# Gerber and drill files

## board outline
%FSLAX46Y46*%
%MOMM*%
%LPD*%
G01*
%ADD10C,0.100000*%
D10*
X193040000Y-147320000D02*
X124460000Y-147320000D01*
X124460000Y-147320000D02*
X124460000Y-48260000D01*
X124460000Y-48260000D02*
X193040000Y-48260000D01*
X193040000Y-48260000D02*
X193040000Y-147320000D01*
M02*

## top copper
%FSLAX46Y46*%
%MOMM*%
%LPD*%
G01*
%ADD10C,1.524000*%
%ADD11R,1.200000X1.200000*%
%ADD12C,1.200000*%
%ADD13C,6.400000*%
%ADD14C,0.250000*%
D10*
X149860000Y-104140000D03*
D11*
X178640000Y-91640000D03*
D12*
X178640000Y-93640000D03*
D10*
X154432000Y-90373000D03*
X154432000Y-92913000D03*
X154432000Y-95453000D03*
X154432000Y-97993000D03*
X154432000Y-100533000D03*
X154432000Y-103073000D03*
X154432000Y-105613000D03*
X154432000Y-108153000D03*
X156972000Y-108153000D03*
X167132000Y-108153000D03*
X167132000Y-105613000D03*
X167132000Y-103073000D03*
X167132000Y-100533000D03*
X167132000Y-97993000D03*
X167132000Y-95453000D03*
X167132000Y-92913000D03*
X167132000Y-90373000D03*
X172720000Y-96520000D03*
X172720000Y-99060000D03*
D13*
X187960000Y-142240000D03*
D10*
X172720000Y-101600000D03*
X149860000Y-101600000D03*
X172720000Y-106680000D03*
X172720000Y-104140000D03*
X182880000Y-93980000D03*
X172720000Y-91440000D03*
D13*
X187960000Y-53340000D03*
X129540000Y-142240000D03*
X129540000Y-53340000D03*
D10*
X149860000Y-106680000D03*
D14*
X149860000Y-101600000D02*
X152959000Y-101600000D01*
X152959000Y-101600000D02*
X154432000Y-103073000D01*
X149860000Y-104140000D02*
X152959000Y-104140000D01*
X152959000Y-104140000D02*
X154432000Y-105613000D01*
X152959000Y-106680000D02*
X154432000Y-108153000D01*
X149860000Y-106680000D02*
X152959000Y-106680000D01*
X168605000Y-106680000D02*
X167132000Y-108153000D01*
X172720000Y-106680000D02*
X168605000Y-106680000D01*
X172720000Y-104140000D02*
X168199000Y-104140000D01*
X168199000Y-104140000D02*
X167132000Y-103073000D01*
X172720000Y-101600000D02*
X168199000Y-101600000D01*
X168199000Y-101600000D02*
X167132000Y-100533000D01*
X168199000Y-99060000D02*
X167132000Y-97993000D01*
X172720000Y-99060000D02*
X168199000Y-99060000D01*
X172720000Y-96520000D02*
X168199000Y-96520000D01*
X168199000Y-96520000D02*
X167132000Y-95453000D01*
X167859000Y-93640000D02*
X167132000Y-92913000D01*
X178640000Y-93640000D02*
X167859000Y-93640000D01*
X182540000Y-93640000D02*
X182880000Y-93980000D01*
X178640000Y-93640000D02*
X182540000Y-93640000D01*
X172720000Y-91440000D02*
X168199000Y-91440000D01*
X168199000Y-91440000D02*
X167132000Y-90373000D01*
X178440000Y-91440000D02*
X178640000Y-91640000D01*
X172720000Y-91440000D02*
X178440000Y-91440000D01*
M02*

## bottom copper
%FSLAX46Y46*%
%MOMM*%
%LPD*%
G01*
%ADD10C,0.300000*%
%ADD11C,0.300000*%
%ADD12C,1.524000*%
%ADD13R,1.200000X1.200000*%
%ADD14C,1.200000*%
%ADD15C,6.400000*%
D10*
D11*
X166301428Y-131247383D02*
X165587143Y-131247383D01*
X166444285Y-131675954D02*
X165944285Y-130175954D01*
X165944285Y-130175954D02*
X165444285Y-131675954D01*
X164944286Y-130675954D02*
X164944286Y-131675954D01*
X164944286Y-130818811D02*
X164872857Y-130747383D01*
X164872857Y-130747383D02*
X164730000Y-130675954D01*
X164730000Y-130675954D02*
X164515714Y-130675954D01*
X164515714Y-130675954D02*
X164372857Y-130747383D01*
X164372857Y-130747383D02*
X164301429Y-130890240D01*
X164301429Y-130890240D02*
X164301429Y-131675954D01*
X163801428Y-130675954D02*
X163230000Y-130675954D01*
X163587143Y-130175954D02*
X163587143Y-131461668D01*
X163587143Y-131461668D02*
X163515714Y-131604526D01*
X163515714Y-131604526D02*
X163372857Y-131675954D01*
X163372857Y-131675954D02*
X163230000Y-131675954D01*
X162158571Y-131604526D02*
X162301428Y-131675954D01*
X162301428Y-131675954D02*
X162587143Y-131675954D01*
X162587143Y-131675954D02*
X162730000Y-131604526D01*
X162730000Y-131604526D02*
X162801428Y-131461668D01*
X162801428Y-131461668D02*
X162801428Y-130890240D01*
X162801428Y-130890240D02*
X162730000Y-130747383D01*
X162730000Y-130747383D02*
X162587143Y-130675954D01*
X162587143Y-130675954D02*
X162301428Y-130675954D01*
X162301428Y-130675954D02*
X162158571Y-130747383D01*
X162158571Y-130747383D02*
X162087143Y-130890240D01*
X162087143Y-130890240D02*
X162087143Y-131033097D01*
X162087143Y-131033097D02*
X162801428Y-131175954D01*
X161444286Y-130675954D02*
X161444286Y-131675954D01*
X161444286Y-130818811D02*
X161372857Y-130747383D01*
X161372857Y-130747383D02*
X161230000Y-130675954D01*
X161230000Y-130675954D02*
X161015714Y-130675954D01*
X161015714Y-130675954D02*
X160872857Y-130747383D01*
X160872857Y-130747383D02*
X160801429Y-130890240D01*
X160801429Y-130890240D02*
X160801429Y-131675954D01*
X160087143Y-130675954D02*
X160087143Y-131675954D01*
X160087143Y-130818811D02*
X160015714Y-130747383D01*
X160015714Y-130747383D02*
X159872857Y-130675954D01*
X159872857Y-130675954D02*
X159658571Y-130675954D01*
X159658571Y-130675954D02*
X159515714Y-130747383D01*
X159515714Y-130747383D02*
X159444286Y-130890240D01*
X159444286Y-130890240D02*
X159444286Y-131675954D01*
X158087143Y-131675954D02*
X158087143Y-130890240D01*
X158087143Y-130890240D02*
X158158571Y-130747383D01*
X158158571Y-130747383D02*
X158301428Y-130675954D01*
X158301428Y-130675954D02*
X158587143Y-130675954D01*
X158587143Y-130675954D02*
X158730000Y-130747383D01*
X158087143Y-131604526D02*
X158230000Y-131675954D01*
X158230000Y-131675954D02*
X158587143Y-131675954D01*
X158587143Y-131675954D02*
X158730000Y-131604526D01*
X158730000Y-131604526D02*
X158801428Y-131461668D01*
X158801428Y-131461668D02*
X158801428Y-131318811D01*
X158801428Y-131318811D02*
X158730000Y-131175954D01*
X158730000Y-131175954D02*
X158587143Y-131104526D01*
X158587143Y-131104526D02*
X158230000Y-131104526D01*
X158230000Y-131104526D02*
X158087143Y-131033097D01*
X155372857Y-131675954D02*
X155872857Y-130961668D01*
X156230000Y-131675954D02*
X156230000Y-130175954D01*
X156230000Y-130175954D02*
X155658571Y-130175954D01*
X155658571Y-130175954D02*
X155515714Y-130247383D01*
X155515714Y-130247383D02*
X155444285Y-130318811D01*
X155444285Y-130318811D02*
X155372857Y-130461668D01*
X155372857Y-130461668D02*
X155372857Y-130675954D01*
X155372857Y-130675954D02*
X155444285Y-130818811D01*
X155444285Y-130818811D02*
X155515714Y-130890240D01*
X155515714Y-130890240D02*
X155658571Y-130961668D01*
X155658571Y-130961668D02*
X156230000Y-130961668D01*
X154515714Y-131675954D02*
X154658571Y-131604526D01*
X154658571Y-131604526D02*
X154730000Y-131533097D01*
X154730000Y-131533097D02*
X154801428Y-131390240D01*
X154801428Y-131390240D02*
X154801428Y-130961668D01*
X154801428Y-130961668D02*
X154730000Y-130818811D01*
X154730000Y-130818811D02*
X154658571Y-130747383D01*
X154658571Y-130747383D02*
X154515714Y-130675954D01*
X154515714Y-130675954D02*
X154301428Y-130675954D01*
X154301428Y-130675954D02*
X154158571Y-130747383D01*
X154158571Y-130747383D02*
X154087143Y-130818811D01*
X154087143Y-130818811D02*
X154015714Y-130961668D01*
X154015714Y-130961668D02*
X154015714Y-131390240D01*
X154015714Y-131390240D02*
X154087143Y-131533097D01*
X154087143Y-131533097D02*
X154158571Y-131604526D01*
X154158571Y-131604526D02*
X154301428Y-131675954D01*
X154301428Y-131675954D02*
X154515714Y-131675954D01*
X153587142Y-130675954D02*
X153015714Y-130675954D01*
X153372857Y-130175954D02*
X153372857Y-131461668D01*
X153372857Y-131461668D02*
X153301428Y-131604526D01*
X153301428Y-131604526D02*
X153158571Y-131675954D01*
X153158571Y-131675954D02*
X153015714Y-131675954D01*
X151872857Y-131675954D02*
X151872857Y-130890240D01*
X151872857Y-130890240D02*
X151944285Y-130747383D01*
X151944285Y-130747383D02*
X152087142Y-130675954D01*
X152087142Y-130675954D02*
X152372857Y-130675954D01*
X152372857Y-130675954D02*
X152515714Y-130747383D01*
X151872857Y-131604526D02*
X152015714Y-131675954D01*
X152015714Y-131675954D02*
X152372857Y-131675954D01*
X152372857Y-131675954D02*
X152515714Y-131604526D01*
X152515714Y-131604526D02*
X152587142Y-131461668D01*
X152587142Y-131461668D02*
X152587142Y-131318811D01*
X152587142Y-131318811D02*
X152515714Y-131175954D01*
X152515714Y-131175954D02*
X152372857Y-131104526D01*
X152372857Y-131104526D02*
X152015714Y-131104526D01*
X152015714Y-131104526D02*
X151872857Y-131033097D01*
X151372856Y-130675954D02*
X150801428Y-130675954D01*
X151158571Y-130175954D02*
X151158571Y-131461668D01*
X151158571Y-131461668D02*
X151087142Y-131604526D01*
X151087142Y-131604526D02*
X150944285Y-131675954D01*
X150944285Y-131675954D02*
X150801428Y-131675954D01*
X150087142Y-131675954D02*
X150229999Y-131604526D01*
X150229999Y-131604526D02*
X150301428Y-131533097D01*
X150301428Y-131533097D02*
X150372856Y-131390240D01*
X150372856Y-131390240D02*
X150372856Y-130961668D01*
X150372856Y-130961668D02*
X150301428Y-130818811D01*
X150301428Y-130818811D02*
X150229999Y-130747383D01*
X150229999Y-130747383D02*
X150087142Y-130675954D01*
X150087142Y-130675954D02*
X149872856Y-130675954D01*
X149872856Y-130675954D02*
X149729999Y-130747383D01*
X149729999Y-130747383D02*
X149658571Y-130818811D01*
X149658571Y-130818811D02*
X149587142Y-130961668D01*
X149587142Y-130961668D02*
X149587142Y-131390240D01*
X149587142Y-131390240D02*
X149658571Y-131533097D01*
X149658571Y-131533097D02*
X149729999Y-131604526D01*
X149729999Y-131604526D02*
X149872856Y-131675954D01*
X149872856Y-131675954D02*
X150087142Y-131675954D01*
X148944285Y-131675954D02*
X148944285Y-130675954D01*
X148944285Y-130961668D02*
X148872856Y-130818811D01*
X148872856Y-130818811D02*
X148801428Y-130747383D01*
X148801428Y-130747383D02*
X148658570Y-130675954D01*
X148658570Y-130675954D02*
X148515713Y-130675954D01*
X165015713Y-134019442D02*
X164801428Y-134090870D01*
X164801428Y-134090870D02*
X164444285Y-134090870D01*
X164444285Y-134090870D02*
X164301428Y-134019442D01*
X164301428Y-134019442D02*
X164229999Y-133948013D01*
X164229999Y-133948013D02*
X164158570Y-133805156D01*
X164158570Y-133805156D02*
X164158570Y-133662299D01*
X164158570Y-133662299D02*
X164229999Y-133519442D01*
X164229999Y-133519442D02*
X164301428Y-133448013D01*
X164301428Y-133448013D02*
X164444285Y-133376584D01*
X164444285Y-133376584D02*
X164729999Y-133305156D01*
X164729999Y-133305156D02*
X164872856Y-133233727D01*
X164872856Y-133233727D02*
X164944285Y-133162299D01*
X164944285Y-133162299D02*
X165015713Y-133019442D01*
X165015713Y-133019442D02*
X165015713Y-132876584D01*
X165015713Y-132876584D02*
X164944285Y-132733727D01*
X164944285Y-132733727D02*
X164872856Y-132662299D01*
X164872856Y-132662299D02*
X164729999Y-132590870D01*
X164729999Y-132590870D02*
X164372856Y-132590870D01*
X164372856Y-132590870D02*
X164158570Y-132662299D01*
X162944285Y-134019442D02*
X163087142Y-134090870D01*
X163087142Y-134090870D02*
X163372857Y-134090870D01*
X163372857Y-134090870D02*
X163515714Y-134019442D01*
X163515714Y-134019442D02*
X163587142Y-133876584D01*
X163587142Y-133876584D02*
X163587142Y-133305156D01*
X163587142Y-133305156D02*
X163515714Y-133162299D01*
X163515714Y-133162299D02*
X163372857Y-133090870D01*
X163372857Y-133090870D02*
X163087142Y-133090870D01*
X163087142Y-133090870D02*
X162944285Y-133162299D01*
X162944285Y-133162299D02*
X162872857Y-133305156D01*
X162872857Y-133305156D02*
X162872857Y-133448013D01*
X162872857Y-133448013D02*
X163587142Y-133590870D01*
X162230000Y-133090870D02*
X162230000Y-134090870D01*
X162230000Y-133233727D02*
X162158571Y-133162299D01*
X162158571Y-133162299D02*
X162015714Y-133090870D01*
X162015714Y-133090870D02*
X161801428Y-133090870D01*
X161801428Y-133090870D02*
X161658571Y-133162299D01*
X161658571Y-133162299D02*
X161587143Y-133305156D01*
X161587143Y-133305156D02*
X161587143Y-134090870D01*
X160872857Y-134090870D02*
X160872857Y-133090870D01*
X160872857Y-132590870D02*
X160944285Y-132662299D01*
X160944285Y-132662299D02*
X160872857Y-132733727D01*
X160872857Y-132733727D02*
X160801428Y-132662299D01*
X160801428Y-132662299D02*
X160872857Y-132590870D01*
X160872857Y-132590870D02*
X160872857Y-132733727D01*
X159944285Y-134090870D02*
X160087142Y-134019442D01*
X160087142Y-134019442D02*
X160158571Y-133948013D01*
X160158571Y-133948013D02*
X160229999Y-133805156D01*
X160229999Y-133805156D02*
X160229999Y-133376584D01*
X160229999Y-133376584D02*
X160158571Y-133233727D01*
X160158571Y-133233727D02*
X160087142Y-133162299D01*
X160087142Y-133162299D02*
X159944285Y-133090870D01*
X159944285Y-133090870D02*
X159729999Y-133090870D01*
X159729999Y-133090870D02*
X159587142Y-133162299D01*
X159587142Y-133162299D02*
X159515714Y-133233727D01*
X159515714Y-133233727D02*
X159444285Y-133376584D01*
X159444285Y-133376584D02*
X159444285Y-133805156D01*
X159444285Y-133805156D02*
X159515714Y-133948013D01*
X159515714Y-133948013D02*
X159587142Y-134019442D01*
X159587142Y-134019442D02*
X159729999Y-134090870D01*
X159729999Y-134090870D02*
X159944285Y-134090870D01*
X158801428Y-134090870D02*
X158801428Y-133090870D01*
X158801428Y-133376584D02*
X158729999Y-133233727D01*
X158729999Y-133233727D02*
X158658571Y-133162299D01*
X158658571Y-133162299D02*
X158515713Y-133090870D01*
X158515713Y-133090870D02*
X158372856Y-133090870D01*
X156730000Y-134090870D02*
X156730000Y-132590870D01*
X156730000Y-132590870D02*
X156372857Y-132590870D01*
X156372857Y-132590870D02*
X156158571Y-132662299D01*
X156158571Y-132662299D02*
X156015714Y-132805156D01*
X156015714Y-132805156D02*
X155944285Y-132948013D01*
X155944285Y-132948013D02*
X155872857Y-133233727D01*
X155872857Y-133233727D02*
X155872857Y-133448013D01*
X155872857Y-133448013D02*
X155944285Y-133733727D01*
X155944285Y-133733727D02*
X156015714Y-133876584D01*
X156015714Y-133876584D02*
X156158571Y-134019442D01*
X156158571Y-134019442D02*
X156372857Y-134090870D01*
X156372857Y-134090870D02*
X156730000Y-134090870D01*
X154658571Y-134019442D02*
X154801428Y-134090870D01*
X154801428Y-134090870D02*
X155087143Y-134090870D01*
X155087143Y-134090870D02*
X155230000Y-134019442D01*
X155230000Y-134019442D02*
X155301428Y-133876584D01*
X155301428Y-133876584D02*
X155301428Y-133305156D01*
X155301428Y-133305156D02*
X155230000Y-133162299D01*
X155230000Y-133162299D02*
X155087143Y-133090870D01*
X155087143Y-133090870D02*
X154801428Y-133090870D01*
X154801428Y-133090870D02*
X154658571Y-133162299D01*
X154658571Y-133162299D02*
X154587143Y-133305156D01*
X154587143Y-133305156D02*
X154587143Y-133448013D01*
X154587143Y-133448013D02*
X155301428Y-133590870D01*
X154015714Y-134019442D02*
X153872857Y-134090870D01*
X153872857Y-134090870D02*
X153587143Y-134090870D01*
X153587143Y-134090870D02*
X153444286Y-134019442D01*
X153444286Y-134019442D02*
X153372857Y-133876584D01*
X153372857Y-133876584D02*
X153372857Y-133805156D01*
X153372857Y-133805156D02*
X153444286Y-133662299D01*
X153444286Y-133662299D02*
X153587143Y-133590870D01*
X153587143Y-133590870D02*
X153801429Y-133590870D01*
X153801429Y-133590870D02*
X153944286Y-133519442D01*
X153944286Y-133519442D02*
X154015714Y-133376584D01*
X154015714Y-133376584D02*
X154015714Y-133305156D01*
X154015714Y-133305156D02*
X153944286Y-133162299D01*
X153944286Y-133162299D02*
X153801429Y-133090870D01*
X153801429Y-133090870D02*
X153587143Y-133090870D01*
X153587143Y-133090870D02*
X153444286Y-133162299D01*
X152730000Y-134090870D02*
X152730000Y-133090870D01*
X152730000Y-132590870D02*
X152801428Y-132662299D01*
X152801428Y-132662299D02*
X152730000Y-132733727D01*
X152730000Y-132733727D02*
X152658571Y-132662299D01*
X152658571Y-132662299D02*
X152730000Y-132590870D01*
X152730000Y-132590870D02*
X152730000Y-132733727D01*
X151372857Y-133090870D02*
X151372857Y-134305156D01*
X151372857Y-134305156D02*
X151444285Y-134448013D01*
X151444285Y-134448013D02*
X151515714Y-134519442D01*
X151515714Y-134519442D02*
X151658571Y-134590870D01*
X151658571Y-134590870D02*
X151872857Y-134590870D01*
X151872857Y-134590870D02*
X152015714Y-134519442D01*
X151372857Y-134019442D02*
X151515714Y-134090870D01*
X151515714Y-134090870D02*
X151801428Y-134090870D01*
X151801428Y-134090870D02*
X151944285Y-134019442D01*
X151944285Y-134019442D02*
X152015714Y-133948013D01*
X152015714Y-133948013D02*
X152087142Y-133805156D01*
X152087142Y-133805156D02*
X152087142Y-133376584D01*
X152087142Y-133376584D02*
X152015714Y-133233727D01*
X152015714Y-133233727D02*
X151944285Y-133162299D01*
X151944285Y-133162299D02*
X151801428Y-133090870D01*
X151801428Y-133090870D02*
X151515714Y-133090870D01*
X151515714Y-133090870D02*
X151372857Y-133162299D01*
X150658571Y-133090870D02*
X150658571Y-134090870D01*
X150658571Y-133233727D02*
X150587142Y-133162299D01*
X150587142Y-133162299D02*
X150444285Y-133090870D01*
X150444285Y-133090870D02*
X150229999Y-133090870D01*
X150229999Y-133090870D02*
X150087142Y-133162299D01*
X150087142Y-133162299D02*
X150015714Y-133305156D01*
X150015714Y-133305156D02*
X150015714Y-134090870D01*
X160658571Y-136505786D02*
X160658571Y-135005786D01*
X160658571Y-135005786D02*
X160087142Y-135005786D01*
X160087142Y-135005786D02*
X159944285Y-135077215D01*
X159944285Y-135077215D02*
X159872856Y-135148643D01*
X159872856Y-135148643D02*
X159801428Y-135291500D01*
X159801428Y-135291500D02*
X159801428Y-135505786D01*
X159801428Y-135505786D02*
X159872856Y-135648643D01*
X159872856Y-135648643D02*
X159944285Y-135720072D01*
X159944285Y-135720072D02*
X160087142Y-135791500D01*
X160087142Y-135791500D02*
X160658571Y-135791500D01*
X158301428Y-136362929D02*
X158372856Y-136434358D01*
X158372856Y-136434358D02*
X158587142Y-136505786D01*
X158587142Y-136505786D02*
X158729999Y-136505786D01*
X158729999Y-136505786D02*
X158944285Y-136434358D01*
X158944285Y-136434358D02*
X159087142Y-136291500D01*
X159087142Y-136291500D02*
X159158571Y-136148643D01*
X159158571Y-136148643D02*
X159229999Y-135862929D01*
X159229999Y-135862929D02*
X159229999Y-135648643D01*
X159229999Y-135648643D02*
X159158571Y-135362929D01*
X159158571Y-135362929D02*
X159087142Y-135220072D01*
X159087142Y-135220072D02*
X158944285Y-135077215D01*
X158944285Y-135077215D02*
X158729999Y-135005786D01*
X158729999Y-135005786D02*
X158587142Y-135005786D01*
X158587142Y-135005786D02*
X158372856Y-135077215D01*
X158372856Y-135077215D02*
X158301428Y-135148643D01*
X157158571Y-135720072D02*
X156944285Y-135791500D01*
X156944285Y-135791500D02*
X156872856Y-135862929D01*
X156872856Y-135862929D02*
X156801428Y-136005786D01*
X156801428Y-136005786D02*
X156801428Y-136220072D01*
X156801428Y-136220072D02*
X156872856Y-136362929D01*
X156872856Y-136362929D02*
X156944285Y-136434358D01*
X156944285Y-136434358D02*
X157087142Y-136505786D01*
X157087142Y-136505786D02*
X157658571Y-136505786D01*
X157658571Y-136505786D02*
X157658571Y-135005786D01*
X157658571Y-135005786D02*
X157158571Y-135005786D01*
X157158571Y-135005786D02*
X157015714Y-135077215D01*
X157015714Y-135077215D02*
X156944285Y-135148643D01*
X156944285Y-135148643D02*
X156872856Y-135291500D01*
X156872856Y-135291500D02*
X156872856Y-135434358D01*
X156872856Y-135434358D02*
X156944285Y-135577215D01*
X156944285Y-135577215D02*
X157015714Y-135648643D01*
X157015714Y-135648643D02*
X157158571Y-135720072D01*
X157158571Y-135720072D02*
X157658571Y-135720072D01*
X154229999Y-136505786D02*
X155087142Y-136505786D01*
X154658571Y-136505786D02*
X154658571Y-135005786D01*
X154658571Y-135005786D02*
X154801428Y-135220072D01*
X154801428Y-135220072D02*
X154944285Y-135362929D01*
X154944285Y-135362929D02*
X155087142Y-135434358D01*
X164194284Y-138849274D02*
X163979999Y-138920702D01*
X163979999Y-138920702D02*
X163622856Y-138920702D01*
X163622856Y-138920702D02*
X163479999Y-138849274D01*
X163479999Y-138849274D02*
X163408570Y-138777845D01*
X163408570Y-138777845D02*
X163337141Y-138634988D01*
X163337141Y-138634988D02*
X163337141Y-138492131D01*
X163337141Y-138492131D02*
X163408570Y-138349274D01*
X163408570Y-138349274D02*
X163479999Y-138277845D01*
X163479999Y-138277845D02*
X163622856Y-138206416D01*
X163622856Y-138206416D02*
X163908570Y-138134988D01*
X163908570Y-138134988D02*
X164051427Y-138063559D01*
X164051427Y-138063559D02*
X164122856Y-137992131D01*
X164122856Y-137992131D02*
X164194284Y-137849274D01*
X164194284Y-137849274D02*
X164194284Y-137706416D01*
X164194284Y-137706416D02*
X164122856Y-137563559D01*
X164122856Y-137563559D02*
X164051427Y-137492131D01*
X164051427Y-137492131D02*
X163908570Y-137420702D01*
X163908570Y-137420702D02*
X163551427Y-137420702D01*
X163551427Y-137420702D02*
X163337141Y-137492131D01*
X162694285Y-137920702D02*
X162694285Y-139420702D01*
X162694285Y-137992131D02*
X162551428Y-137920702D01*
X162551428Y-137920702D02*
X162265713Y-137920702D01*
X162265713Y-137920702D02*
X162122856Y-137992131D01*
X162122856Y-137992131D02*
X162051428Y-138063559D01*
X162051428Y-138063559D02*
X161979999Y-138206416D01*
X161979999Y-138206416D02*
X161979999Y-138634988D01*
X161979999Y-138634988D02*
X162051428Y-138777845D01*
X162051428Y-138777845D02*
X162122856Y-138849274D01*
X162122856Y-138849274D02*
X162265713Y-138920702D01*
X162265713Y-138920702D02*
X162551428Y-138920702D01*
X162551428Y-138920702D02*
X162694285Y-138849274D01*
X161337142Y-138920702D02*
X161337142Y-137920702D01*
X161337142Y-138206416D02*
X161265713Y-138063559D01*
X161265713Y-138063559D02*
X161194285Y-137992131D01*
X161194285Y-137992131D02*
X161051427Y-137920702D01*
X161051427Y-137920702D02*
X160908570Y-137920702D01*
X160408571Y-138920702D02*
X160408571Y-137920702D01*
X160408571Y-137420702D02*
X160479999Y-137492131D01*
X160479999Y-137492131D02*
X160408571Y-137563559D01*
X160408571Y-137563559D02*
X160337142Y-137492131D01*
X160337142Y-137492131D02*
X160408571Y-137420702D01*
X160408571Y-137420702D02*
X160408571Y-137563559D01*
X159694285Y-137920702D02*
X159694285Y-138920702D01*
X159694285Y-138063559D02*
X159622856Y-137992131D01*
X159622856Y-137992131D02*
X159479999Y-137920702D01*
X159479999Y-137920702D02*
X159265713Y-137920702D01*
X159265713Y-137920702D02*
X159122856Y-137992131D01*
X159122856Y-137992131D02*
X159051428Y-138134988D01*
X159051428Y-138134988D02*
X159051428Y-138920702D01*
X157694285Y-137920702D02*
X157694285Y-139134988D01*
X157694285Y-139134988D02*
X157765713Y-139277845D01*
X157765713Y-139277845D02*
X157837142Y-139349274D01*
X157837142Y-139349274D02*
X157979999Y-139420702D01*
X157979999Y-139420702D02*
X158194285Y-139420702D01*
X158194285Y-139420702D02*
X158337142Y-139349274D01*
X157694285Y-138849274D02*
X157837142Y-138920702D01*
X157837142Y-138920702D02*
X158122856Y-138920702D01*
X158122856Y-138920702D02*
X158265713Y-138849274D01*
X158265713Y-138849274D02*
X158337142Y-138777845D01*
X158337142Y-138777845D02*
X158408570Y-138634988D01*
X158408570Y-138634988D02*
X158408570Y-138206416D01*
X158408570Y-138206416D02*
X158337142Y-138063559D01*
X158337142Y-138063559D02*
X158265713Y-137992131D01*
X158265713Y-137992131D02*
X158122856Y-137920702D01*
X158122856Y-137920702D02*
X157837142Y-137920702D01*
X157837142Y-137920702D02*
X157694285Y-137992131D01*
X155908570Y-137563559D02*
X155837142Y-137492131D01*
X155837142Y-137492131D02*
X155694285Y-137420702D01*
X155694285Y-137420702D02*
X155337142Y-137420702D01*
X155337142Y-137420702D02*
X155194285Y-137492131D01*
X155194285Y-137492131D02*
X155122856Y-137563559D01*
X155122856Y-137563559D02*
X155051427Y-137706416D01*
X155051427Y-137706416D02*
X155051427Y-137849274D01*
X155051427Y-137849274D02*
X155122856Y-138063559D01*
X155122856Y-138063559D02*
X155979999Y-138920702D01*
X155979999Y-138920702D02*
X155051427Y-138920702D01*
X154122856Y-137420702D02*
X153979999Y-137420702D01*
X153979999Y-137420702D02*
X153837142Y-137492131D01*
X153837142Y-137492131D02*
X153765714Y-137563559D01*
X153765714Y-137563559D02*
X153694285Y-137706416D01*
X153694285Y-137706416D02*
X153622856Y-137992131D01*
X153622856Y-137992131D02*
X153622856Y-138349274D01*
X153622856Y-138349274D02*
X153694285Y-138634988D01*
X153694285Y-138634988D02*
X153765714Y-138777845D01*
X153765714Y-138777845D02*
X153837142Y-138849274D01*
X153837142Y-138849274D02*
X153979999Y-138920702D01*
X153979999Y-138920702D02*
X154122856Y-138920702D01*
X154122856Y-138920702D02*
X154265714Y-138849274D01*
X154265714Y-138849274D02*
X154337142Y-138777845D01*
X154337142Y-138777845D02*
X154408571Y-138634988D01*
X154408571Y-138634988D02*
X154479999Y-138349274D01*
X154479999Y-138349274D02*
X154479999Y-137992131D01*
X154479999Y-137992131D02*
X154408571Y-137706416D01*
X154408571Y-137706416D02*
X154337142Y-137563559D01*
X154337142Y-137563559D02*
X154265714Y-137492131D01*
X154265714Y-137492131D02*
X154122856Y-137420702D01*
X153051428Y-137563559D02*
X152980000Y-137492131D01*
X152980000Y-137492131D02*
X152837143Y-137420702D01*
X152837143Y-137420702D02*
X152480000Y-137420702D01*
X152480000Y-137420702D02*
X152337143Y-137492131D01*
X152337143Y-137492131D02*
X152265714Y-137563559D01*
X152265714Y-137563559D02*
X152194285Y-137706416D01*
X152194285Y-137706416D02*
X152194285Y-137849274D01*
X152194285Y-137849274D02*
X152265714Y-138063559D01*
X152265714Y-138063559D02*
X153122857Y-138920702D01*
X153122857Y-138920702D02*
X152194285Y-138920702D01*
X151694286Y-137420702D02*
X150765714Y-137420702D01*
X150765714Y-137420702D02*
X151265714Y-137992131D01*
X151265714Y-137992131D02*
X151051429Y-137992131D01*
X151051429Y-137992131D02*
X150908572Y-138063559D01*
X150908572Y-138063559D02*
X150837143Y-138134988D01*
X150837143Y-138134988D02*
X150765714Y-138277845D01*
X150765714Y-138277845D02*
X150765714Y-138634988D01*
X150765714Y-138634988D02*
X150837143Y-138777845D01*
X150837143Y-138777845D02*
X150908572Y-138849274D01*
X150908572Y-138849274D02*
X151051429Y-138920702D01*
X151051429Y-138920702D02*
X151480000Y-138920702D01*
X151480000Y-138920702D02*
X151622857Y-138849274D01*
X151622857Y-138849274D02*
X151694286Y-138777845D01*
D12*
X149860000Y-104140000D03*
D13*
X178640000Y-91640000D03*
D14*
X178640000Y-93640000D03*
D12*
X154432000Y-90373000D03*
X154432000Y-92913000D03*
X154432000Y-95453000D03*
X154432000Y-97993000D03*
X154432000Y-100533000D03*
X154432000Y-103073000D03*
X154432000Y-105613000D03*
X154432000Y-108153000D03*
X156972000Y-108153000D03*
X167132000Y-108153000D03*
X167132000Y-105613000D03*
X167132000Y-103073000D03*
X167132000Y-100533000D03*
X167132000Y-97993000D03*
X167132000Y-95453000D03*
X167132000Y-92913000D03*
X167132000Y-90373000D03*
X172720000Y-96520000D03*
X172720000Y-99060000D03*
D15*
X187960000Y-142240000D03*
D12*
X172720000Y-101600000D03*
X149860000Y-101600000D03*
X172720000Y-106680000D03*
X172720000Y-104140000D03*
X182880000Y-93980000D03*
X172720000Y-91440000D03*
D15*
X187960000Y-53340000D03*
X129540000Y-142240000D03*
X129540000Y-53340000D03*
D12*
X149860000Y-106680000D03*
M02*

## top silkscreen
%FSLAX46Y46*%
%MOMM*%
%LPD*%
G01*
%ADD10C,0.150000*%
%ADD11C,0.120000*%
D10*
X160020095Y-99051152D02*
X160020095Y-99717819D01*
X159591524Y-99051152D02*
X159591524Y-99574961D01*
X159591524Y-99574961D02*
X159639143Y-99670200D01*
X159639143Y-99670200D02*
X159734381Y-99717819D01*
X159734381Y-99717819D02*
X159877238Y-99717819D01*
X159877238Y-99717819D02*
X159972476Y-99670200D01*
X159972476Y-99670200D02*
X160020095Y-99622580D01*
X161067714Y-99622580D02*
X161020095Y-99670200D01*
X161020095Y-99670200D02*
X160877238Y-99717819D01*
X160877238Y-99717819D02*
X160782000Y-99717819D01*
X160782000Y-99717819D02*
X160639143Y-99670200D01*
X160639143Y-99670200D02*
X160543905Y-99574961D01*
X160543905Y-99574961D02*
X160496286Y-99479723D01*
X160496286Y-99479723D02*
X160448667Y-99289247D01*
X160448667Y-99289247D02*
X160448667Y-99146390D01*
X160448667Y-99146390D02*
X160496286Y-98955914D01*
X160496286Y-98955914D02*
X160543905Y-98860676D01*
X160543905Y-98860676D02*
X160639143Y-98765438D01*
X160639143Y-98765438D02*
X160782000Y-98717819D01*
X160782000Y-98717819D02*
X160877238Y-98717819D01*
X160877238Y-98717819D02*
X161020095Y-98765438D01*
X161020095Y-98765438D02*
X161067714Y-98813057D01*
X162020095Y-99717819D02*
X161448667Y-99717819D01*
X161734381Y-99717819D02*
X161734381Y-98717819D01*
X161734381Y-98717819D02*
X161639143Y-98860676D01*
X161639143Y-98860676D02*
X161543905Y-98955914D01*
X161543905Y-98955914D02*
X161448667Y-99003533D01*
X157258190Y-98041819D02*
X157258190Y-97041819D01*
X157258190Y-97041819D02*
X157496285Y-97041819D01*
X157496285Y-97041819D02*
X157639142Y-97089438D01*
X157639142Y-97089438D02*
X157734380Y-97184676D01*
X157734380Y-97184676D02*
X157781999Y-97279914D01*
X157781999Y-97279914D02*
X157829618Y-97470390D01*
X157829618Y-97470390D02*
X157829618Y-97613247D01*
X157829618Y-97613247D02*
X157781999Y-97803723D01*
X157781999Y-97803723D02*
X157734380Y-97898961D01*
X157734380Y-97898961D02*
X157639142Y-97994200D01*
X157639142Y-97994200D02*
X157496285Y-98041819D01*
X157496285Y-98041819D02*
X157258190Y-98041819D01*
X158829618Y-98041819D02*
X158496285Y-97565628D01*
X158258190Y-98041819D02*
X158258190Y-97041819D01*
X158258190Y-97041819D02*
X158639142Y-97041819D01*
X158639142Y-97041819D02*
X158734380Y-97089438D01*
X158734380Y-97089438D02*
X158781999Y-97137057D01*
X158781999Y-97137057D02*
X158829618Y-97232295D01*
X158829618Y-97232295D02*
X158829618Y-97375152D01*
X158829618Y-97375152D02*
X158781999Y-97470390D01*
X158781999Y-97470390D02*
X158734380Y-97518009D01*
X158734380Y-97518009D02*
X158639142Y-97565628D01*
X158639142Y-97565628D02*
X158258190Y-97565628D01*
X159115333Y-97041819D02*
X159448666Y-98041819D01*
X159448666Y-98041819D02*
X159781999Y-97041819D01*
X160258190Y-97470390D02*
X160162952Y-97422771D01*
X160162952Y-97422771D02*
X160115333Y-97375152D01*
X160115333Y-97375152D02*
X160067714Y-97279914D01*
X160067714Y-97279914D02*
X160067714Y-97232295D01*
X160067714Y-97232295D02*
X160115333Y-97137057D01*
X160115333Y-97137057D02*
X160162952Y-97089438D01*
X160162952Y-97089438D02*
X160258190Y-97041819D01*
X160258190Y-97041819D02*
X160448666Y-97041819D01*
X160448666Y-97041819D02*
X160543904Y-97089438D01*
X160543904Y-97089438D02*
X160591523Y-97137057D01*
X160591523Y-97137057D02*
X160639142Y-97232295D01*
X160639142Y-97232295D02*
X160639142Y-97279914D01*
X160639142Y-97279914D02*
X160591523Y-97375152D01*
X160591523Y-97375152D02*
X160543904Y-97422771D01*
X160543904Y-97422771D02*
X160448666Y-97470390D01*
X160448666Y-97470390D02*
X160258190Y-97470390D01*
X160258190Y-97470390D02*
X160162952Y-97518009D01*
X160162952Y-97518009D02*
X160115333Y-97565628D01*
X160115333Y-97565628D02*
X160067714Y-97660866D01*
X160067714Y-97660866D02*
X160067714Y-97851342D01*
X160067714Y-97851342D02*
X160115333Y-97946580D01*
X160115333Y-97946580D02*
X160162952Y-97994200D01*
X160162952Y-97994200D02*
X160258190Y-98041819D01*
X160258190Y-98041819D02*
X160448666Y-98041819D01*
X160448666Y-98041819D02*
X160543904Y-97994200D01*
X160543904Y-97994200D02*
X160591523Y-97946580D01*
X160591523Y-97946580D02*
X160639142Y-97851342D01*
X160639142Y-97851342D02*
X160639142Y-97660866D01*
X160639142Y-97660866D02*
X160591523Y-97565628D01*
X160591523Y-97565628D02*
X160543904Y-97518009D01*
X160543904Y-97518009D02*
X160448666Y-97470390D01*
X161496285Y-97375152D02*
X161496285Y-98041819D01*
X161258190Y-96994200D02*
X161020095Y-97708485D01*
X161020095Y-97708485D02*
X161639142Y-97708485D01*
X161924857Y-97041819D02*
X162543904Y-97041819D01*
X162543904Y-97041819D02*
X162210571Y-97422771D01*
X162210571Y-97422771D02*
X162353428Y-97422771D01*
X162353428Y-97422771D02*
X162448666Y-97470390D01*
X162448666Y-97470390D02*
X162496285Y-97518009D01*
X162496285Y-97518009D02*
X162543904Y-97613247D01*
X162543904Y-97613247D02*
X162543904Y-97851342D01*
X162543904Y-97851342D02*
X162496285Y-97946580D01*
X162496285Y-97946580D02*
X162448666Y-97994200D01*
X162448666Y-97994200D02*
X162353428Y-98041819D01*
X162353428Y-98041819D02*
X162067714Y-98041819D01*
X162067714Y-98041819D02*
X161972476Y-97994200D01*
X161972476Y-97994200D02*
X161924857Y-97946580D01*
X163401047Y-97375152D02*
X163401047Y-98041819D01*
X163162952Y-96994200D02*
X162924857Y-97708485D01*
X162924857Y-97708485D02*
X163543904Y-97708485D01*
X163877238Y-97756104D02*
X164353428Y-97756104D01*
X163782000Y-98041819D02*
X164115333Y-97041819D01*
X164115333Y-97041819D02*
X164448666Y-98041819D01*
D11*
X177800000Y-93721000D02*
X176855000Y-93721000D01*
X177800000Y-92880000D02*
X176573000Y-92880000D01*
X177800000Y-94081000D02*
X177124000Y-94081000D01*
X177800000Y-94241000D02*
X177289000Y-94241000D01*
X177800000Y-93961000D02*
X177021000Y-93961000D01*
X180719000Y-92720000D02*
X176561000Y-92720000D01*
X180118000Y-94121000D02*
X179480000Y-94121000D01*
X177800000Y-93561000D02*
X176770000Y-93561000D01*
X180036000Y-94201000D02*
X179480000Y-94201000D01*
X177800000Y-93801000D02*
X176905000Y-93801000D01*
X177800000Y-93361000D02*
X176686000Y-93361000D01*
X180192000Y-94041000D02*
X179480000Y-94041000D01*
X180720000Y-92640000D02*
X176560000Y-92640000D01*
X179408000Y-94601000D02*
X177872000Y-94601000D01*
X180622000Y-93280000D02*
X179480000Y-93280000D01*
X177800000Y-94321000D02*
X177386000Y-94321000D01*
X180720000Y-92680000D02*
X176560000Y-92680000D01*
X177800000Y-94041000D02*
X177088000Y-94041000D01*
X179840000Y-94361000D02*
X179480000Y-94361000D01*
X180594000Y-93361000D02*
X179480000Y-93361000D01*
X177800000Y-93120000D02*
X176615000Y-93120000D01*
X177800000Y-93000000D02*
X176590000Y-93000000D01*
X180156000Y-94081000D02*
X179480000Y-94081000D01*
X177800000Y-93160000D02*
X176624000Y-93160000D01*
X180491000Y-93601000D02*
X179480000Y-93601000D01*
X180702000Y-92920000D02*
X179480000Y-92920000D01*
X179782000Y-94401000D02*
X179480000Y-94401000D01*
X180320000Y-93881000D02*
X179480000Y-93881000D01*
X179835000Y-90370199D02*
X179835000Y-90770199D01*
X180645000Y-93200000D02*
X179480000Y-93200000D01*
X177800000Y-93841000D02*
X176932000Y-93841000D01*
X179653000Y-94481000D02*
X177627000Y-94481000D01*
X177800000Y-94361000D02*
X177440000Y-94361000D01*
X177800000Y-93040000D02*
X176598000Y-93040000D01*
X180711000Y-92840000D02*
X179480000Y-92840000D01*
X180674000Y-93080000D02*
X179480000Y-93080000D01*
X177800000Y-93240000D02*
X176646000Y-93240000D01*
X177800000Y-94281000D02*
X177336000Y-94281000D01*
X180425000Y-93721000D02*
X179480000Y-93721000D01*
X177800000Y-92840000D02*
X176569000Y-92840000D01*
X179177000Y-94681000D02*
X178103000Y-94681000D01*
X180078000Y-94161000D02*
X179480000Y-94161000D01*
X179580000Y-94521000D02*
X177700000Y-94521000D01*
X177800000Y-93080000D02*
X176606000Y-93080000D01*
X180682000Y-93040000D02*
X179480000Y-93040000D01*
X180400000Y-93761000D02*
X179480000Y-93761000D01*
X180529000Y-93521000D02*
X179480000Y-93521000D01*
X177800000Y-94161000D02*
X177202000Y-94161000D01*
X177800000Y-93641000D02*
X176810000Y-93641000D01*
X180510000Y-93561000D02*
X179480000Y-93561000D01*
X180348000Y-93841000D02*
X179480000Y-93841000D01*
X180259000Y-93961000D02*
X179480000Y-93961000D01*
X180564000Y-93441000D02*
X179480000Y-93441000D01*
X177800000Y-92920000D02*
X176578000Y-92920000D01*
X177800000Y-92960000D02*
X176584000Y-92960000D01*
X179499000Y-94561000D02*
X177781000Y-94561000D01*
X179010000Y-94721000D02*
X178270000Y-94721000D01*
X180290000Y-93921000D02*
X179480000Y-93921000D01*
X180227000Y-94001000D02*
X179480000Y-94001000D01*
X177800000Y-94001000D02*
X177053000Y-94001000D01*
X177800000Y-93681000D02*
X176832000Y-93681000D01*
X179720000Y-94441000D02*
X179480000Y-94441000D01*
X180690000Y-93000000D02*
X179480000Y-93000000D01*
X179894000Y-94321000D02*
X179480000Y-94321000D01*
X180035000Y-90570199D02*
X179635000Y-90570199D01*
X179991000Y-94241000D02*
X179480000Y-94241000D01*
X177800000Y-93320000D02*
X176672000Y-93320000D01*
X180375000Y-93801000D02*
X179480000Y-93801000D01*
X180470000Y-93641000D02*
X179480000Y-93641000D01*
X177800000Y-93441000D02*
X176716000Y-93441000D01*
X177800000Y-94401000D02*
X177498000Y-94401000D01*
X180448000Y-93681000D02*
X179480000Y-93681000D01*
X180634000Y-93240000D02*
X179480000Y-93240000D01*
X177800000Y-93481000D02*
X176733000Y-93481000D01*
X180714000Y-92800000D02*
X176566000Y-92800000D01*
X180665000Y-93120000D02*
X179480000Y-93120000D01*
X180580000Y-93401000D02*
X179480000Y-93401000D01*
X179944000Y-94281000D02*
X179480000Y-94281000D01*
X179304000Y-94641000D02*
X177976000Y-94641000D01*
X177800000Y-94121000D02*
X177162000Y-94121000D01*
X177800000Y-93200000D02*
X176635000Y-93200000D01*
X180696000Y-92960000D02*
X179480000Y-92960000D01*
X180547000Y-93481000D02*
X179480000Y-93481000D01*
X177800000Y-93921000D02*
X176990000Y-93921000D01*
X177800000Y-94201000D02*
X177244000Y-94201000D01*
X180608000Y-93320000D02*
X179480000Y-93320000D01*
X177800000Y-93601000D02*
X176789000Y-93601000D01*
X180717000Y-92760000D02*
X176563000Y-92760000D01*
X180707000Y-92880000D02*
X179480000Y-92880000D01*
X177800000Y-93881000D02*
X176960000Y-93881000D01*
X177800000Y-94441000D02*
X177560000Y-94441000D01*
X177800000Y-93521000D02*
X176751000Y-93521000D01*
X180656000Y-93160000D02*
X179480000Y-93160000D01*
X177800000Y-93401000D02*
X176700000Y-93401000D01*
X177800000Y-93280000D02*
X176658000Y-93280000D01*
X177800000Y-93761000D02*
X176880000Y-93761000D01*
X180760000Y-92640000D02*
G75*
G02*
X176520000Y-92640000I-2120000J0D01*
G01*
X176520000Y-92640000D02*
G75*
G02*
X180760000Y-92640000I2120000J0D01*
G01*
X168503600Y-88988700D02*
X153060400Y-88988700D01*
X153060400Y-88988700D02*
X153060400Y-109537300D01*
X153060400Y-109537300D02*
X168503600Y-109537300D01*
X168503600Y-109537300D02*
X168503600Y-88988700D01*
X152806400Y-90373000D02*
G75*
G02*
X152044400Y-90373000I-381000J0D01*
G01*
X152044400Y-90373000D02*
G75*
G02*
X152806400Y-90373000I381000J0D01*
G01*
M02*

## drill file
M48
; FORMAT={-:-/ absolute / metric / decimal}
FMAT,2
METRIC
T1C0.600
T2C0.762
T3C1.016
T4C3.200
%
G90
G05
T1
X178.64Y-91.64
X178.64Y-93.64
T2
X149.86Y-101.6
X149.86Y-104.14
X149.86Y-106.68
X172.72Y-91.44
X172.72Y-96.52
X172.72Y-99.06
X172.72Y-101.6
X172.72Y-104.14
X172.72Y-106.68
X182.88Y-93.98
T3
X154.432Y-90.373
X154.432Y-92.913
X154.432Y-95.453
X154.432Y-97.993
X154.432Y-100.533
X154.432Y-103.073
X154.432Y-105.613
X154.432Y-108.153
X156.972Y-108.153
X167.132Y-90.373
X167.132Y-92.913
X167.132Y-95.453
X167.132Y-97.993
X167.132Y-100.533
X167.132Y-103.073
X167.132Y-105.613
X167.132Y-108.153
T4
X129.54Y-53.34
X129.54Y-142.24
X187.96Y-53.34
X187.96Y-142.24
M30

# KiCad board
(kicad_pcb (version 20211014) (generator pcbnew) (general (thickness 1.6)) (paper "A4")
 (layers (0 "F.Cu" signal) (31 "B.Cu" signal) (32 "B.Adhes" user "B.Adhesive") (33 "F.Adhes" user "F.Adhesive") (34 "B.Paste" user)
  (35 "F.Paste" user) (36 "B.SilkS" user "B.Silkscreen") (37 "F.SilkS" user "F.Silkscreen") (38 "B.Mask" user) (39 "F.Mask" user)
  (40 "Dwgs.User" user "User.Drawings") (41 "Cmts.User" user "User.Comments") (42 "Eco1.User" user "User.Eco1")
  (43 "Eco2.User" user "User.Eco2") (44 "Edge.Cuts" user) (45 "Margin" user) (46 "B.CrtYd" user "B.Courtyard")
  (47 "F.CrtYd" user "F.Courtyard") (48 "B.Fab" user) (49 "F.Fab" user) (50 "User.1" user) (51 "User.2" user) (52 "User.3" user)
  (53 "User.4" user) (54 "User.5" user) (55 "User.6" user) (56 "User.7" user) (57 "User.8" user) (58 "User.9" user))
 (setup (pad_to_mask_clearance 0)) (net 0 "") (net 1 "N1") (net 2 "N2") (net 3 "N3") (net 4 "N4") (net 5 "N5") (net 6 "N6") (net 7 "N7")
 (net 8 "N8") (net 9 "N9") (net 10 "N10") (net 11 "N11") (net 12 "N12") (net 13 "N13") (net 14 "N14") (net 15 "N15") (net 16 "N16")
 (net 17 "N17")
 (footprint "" (layer "F.Cu") (at 149.86 104.14)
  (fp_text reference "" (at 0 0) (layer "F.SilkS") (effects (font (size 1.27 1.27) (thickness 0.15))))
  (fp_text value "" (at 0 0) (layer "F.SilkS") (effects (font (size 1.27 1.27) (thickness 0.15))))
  (pad "1" thru_hole circle (at 0 0) (size 1.524 1.524) (drill 0.762) (layers *.Cu *.Mask) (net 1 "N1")))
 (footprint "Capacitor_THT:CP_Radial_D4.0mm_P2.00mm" (layer "F.Cu") (at 178.64 91.64 -90)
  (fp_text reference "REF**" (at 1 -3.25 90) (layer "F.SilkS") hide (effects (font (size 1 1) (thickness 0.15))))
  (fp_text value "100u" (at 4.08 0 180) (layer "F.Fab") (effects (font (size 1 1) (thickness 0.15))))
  (fp_line (start 2.081 0.84) (end 2.081 1.785) (layer "F.SilkS") (width 0.12))
  (fp_line (start 1.24 0.84) (end 1.24 2.067) (layer "F.SilkS") (width 0.12))
  (fp_line (start 2.441 0.84) (end 2.441 1.516) (layer "F.SilkS") (width 0.12))
  (fp_line (start 2.601 0.84) (end 2.601 1.351) (layer "F.SilkS") (width 0.12))
  (fp_line (start 2.321 0.84) (end 2.321 1.619) (layer "F.SilkS") (width 0.12))
  (fp_line (start 1.08 -2.079) (end 1.08 2.079) (layer "F.SilkS") (width 0.12))
  (fp_line (start 2.481 -1.478) (end 2.481 -0.84) (layer "F.SilkS") (width 0.12))
  (fp_line (start 1.921 0.84) (end 1.921 1.87) (layer "F.SilkS") (width 0.12))
  (fp_line (start 2.561 -1.396) (end 2.561 -0.84) (layer "F.SilkS") (width 0.12))
  (fp_line (start 2.161 0.84) (end 2.161 1.735) (layer "F.SilkS") (width 0.12))
  (fp_line (start 1.721 0.84) (end 1.721 1.954) (layer "F.SilkS") (width 0.12))
  (fp_line (start 2.401 -1.552) (end 2.401 -0.84) (layer "F.SilkS") (width 0.12))
  (fp_line (start 1 -2.08) (end 1 2.08) (layer "F.SilkS") (width 0.12))
  (fp_line (start 2.961 -0.768) (end 2.961 0.768) (layer "F.SilkS") (width 0.12))
  (fp_line (start 1.64 -1.982) (end 1.64 -0.84) (layer "F.SilkS") (width 0.12))
  (fp_line (start 2.681 0.84) (end 2.681 1.254) (layer "F.SilkS") (width 0.12))
  (fp_line (start 1.04 -2.08) (end 1.04 2.08) (layer "F.SilkS") (width 0.12))
  (fp_line (start 2.401 0.84) (end 2.401 1.552) (layer "F.SilkS") (width 0.12))
  (fp_line (start 2.721 -1.2) (end 2.721 -0.84) (layer "F.SilkS") (width 0.12))
  (fp_line (start 1.721 -1.954) (end 1.721 -0.84) (layer "F.SilkS") (width 0.12))
  (fp_line (start 1.48 0.84) (end 1.48 2.025) (layer "F.SilkS") (width 0.12))
  (fp_line (start 1.36 0.84) (end 1.36 2.05) (layer "F.SilkS") (width 0.12))
  (fp_line (start 2.441 -1.516) (end 2.441 -0.84) (layer "F.SilkS") (width 0.12))
  (fp_line (start 1.52 0.84) (end 1.52 2.016) (layer "F.SilkS") (width 0.12))
  (fp_line (start 1.961 -1.851) (end 1.961 -0.84) (layer "F.SilkS") (width 0.12))
  (fp_line (start 1.28 -2.062) (end 1.28 -0.84) (layer "F.SilkS") (width 0.12))
  (fp_line (start 2.761 -1.142) (end 2.761 -0.84) (layer "F.SilkS") (width 0.12))
  (fp_line (start 2.241 -1.68) (end 2.241 -0.84) (layer "F.SilkS") (width 0.12))
  (fp_line (start -1.269801 -1.195) (end -0.869801 -1.195) (layer "F.SilkS") (width 0.12))
  (fp_line (start 1.56 -2.005) (end 1.56 -0.84) (layer "F.SilkS") (width 0.12))
  (fp_line (start 2.201 0.84) (end 2.201 1.708) (layer "F.SilkS") (width 0.12))
  (fp_line (start 2.841 -1.013) (end 2.841 1.013) (layer "F.SilkS") (width 0.12))
  (fp_line (start 2.721 0.84) (end 2.721 1.2) (layer "F.SilkS") (width 0.12))
  (fp_line (start 1.4 0.84) (end 1.4 2.042) (layer "F.SilkS") (width 0.12))
  (fp_line (start 1.2 -2.071) (end 1.2 -0.84) (layer "F.SilkS") (width 0.12))
  (fp_line (start 1.44 -2.034) (end 1.44 -0.84) (layer "F.SilkS") (width 0.12))
  (fp_line (start 1.6 0.84) (end 1.6 1.994) (layer "F.SilkS") (width 0.12))
  (fp_line (start 2.641 0.84) (end 2.641 1.304) (layer "F.SilkS") (width 0.12))
  (fp_line (start 2.081 -1.785) (end 2.081 -0.84) (layer "F.SilkS") (width 0.12))
  (fp_line (start 1.2 0.84) (end 1.2 2.071) (layer "F.SilkS") (width 0.12))
  (fp_line (start 3.041 -0.537) (end 3.041 0.537) (layer "F.SilkS") (width 0.12))
  (fp_line (start 2.521 -1.438) (end 2.521 -0.84) (layer "F.SilkS") (width 0.12))
  (fp_line (start 2.881 -0.94) (end 2.881 0.94) (layer "F.SilkS") (width 0.12))
  (fp_line (start 1.44 0.84) (end 1.44 2.034) (layer "F.SilkS") (width 0.12))
  (fp_line (start 1.4 -2.042) (end 1.4 -0.84) (layer "F.SilkS") (width 0.12))
  (fp_line (start 2.121 -1.76) (end 2.121 -0.84) (layer "F.SilkS") (width 0.12))
  (fp_line (start 1.881 -1.889) (end 1.881 -0.84) (layer "F.SilkS") (width 0.12))
  (fp_line (start 2.521 0.84) (end 2.521 1.438) (layer "F.SilkS") (width 0.12))
  (fp_line (start 2.001 0.84) (end 2.001 1.83) (layer "F.SilkS") (width 0.12))
  (fp_line (start 1.921 -1.87) (end 1.921 -0.84) (layer "F.SilkS") (width 0.12))
  (fp_line (start 2.201 -1.708) (end 2.201 -0.84) (layer "F.SilkS") (width 0.12))
  (fp_line (start 2.321 -1.619) (end 2.321 -0.84) (layer "F.SilkS") (width 0.12))
  (fp_line (start 1.801 -1.924) (end 1.801 -0.84) (layer "F.SilkS") (width 0.12))
  (fp_line (start 1.28 0.84) (end 1.28 2.062) (layer "F.SilkS") (width 0.12))
  (fp_line (start 1.32 0.84) (end 1.32 2.056) (layer "F.SilkS") (width 0.12))
  (fp_line (start 2.921 -0.859) (end 2.921 0.859) (layer "F.SilkS") (width 0.12))
  (fp_line (start 3.081 -0.37) (end 3.081 0.37) (layer "F.SilkS") (width 0.12))
  (fp_line (start 2.281 -1.65) (end 2.281 -0.84) (layer "F.SilkS") (width 0.12))
  (fp_line (start 2.361 -1.587) (end 2.361 -0.84) (layer "F.SilkS") (width 0.12))
  (fp_line (start 2.361 0.84) (end 2.361 1.587) (layer "F.SilkS") (width 0.12))
  (fp_line (start 2.041 0.84) (end 2.041 1.808) (layer "F.SilkS") (width 0.12))
  (fp_line (start 2.801 -1.08) (end 2.801 -0.84) (layer "F.SilkS") (width 0.12))
  (fp_line (start 1.36 -2.05) (end 1.36 -0.84) (layer "F.SilkS") (width 0.12))
  (fp_line (start 2.681 -1.254) (end 2.681 -0.84) (layer "F.SilkS") (width 0.12))
  (fp_line (start -1.069801 -1.395) (end -1.069801 -0.995) (layer "F.SilkS") (width 0.12))
  (fp_line (start 2.601 -1.351) (end 2.601 -0.84) (layer "F.SilkS") (width 0.12))
  (fp_line (start 1.68 0.84) (end 1.68 1.968) (layer "F.SilkS") (width 0.12))
  (fp_line (start 2.161 -1.735) (end 2.161 -0.84) (layer "F.SilkS") (width 0.12))
  (fp_line (start 2.001 -1.83) (end 2.001 -0.84) (layer "F.SilkS") (width 0.12))
  (fp_line (start 1.801 0.84) (end 1.801 1.924) (layer "F.SilkS") (width 0.12))
  (fp_line (start 2.761 0.84) (end 2.761 1.142) (layer "F.SilkS") (width 0.12))
  (fp_line (start 2.041 -1.808) (end 2.041 -0.84) (layer "F.SilkS") (width 0.12))
  (fp_line (start 1.6 -1.994) (end 1.6 -0.84) (layer "F.SilkS") (width 0.12))
  (fp_line (start 1.841 0.84) (end 1.841 1.907) (layer "F.SilkS") (width 0.12))
  (fp_line (start 1.16 -2.074) (end 1.16 2.074) (layer "F.SilkS") (width 0.12))
  (fp_line (start 1.48 -2.025) (end 1.48 -0.84) (layer "F.SilkS") (width 0.12))
  (fp_line (start 1.761 -1.94) (end 1.761 -0.84) (layer "F.SilkS") (width 0.12))
  (fp_line (start 2.641 -1.304) (end 2.641 -0.84) (layer "F.SilkS") (width 0.12))
  (fp_line (start 3.001 -0.664) (end 3.001 0.664) (layer "F.SilkS") (width 0.12))
  (fp_line (start 2.481 0.84) (end 2.481 1.478) (layer "F.SilkS") (width 0.12))
  (fp_line (start 1.56 0.84) (end 1.56 2.005) (layer "F.SilkS") (width 0.12))
  (fp_line (start 1.32 -2.056) (end 1.32 -0.84) (layer "F.SilkS") (width 0.12))
  (fp_line (start 1.841 -1.907) (end 1.841 -0.84) (layer "F.SilkS") (width 0.12))
  (fp_line (start 2.281 0.84) (end 2.281 1.65) (layer "F.SilkS") (width 0.12))
  (fp_line (start 2.561 0.84) (end 2.561 1.396) (layer "F.SilkS") (width 0.12))
  (fp_line (start 1.68 -1.968) (end 1.68 -0.84) (layer "F.SilkS") (width 0.12))
  (fp_line (start 1.961 0.84) (end 1.961 1.851) (layer "F.SilkS") (width 0.12))
  (fp_line (start 1.12 -2.077) (end 1.12 2.077) (layer "F.SilkS") (width 0.12))
  (fp_line (start 1.24 -2.067) (end 1.24 -0.84) (layer "F.SilkS") (width 0.12))
  (fp_line (start 2.241 0.84) (end 2.241 1.68) (layer "F.SilkS") (width 0.12))
  (fp_line (start 2.801 0.84) (end 2.801 1.08) (layer "F.SilkS") (width 0.12))
  (fp_line (start 1.881 0.84) (end 1.881 1.889) (layer "F.SilkS") (width 0.12))
  (fp_line (start 1.52 -2.016) (end 1.52 -0.84) (layer "F.SilkS") (width 0.12))
  (fp_line (start 1.761 0.84) (end 1.761 1.94) (layer "F.SilkS") (width 0.12))
  (fp_line (start 1.64 0.84) (end 1.64 1.982) (layer "F.SilkS") (width 0.12))
  (fp_line (start 2.121 0.84) (end 2.121 1.76) (layer "F.SilkS") (width 0.12))
  (fp_circle (center 1 0) (end 3.12 0) (layer "F.SilkS") (width 0.12) (fill none))
  (pad "1" thru_hole rect (at 0 0 270) (size 1.2 1.2) (drill 0.6) (layers *.Cu *.Mask) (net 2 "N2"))
  (pad "2" thru_hole circle (at 2 0 270) (size 1.2 1.2) (drill 0.6) (layers *.Cu *.Mask) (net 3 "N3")))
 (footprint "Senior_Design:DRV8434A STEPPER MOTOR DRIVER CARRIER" (layer "F.Cu") (at 154.432 90.373)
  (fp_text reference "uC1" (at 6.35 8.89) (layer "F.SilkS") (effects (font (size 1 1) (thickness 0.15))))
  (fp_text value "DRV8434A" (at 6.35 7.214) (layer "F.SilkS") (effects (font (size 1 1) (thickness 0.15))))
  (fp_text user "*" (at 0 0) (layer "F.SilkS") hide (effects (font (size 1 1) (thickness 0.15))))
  (fp_line (start 14.0716 -1.3843) (end -1.3716 -1.3843) (layer "F.SilkS") (width 0.12))
  (fp_line (start -1.3716 -1.3843) (end -1.3716 19.1643) (layer "F.SilkS") (width 0.12))
  (fp_line (start -1.3716 19.1643) (end 14.0716 19.1643) (layer "F.SilkS") (width 0.12))
  (fp_line (start 14.0716 19.1643) (end 14.0716 -1.3843) (layer "F.SilkS") (width 0.12))
  (fp_circle (center -2.0066 0) (end -1.6256 0) (layer "F.SilkS") (width 0.12) (fill none))
  (pad "1" thru_hole circle (at 0 0) (size 1.524 1.524) (drill 1.016) (layers *.Cu *.Mask) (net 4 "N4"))
  (pad "2" thru_hole circle (at 0 2.54) (size 1.524 1.524) (drill 1.016) (layers *.Cu *.Mask) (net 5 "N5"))
  (pad "3" thru_hole circle (at 0 5.08) (size 1.524 1.524) (drill 1.016) (layers *.Cu *.Mask) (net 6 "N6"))
  (pad "4" thru_hole circle (at 0 7.62) (size 1.524 1.524) (drill 1.016) (layers *.Cu *.Mask) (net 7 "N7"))
  (pad "5" thru_hole circle (at 0 10.16) (size 1.524 1.524) (drill 1.016) (layers *.Cu *.Mask) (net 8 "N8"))
  (pad "6" thru_hole circle (at 0 12.7) (size 1.524 1.524) (drill 1.016) (layers *.Cu *.Mask) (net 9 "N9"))
  (pad "7" thru_hole circle (at 0 15.24) (size 1.524 1.524) (drill 1.016) (layers *.Cu *.Mask) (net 1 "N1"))
  (pad "8" thru_hole circle (at 0 17.78) (size 1.524 1.524) (drill 1.016) (layers *.Cu *.Mask) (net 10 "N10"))
  (pad "9" thru_hole circle (at 2.54 17.78) (size 1.524 1.524) (drill 1.016) (layers *.Cu *.Mask) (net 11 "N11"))
  (pad "10" thru_hole circle (at 12.7 17.78) (size 1.524 1.524) (drill 1.016) (layers *.Cu *.Mask) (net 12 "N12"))
  (pad "11" thru_hole circle (at 12.7 15.24) (size 1.524 1.524) (drill 1.016) (layers *.Cu *.Mask) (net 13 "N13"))
  (pad "12" thru_hole circle (at 12.7 12.7) (size 1.524 1.524) (drill 1.016) (layers *.Cu *.Mask) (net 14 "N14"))
  (pad "13" thru_hole circle (at 12.7 10.16) (size 1.524 1.524) (drill 1.016) (layers *.Cu *.Mask) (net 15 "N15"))
  (pad "14" thru_hole circle (at 12.7 7.62) (size 1.524 1.524) (drill 1.016) (layers *.Cu *.Mask) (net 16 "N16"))
  (pad "15" thru_hole circle (at 12.7 5.08) (size 1.524 1.524) (drill 1.016) (layers *.Cu *.Mask) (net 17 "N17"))
  (pad "16" thru_hole circle (at 12.7 2.54) (size 1.524 1.524) (drill 1.016) (layers *.Cu *.Mask) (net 3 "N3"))
  (pad "17" thru_hole circle (at 12.7 0) (size 1.524 1.524) (drill 1.016) (layers *.Cu *.Mask) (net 2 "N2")))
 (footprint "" (layer "F.Cu") (at 172.72 96.52)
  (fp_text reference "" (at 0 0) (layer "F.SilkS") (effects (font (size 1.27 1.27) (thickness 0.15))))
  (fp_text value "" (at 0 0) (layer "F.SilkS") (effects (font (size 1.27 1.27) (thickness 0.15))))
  (pad "1" thru_hole circle (at 0 0) (size 1.524 1.524) (drill 0.762) (layers *.Cu *.Mask) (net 17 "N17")))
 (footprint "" (layer "F.Cu") (at 172.72 99.06)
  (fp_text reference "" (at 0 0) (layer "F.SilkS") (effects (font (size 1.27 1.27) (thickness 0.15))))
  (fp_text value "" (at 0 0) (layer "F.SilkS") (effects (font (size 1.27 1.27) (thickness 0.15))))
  (pad "1" thru_hole circle (at 0 0) (size 1.524 1.524) (drill 0.762) (layers *.Cu *.Mask) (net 16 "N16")))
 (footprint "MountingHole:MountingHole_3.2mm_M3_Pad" (layer "F.Cu") (at 187.96 142.24)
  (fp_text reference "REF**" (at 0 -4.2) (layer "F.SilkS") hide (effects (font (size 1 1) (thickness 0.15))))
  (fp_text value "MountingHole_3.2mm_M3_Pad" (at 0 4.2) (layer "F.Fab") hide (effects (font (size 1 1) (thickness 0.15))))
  (pad "1" thru_hole circle (at 0 0) (size 6.4 6.4) (drill 3.2) (layers F&B.Cu *.Mask)))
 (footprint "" (layer "F.Cu") (at 172.72 101.6)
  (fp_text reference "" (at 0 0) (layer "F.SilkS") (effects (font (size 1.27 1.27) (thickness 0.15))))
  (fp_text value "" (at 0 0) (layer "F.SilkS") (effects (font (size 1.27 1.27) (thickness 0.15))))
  (pad "1" thru_hole circle (at 0 0) (size 1.524 1.524) (drill 0.762) (layers *.Cu *.Mask) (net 15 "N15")))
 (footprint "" (layer "F.Cu") (at 149.86 101.6)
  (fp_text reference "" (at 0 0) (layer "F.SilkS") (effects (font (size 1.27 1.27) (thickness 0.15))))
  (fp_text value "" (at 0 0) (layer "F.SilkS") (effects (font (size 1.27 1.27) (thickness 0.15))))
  (pad "1" thru_hole circle (at 0 0) (size 1.524 1.524) (drill 0.762) (layers *.Cu *.Mask) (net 9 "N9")))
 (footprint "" (layer "F.Cu") (at 172.72 106.68)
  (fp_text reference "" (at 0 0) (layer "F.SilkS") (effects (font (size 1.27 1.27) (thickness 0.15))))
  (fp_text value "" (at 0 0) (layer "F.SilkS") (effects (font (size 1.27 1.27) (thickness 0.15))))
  (pad "1" thru_hole circle (at 0 0) (size 1.524 1.524) (drill 0.762) (layers *.Cu *.Mask) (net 12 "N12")))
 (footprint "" (layer "F.Cu") (at 172.72 104.14)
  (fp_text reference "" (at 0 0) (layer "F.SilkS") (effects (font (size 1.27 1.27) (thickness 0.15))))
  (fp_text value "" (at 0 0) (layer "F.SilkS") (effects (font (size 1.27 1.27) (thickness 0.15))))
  (pad "1" thru_hole circle (at 0 0) (size 1.524 1.524) (drill 0.762) (layers *.Cu *.Mask) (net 14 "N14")))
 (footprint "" (layer "F.Cu") (at 182.88 93.98)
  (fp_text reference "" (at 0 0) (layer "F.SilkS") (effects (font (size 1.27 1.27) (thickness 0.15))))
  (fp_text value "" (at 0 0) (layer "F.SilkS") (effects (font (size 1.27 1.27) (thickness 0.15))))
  (pad "1" thru_hole circle (at 0 0) (size 1.524 1.524) (drill 0.762) (layers *.Cu *.Mask) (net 3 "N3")))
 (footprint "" (layer "F.Cu") (at 172.72 91.44)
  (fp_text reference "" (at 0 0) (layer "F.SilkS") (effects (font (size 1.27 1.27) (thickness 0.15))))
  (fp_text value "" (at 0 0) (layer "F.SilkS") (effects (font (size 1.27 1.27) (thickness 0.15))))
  (pad "1" thru_hole circle (at 0 0) (size 1.524 1.524) (drill 0.762) (layers *.Cu *.Mask) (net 2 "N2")))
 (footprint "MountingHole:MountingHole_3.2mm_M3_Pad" (layer "F.Cu") (at 187.96 53.34)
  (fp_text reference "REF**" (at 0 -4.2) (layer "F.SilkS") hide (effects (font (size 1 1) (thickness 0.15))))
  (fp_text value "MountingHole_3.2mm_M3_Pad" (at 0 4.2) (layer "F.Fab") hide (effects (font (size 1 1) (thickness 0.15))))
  (pad "1" thru_hole circle (at 0 0) (size 6.4 6.4) (drill 3.2) (layers F&B.Cu *.Mask)))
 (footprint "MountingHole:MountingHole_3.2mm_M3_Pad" (layer "F.Cu") (at 129.54 142.24)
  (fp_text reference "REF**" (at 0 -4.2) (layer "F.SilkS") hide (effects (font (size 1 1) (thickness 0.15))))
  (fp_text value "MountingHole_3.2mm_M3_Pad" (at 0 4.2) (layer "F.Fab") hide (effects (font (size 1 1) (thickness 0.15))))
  (pad "1" thru_hole circle (at 0 0) (size 6.4 6.4) (drill 3.2) (layers F&B.Cu *.Mask)))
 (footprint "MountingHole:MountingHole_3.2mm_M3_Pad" (layer "F.Cu") (at 129.54 53.34)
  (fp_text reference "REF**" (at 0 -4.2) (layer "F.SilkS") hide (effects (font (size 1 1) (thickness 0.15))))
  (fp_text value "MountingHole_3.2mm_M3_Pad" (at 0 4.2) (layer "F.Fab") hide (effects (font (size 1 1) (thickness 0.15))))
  (pad "1" thru_hole circle (at 0 0) (size 6.4 6.4) (drill 3.2) (layers *.Cu *.Mask)))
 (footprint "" (layer "F.Cu") (at 149.86 106.68)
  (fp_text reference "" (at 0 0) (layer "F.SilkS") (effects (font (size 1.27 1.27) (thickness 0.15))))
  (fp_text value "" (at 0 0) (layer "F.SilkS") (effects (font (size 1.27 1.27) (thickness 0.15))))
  (pad "1" thru_hole circle (at 0 0) (size 1.524 1.524) (drill 0.762) (layers *.Cu *.Mask) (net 10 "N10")))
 (gr_line (start 193.04 147.32) (end 124.46 147.32) (layer "Edge.Cuts") (width 0.1))
 (gr_line (start 124.46 147.32) (end 124.46 48.26) (layer "Edge.Cuts") (width 0.1))
 (gr_line (start 124.46 48.26) (end 193.04 48.26) (layer "Edge.Cuts") (width 0.1))
 (gr_line (start 193.04 48.26) (end 193.04 147.32) (layer "Edge.Cuts") (width 0.1))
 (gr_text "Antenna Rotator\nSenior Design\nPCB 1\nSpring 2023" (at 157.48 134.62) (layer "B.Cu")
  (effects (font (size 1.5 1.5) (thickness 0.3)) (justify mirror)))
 (segment (start 149.86 101.6) (end 152.959 101.6) (width 0.25) (layer "F.Cu") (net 9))
 (segment (start 152.959 101.6) (end 154.432 103.073) (width 0.25) (layer "F.Cu") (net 9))
 (segment (start 149.86 104.14) (end 152.959 104.14) (width 0.25) (layer "F.Cu") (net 1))
 (segment (start 152.959 104.14) (end 154.432 105.613) (width 0.25) (layer "F.Cu") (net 1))
 (segment (start 152.959 106.68) (end 154.432 108.153) (width 0.25) (layer "F.Cu") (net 10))
 (segment (start 149.86 106.68) (end 152.959 106.68) (width 0.25) (layer "F.Cu") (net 10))
 (segment (start 168.605 106.68) (end 167.132 108.153) (width 0.25) (layer "F.Cu") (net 12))
 (segment (start 172.72 106.68) (end 168.605 106.68) (width 0.25) (layer "F.Cu") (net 12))
 (segment (start 172.72 104.14) (end 168.199 104.14) (width 0.25) (layer "F.Cu") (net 14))
 (segment (start 168.199 104.14) (end 167.132 103.073) (width 0.25) (layer "F.Cu") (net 14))
 (segment (start 172.72 101.6) (end 168.199 101.6) (width 0.25) (layer "F.Cu") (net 15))
 (segment (start 168.199 101.6) (end 167.132 100.533) (width 0.25) (layer "F.Cu") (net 15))
 (segment (start 168.199 99.06) (end 167.132 97.993) (width 0.25) (layer "F.Cu") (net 16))
 (segment (start 172.72 99.06) (end 168.199 99.06) (width 0.25) (layer "F.Cu") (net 16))
 (segment (start 172.72 96.52) (end 168.199 96.52) (width 0.25) (layer "F.Cu") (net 17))
 (segment (start 168.199 96.52) (end 167.132 95.453) (width 0.25) (layer "F.Cu") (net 17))
 (segment (start 167.859 93.64) (end 167.132 92.913) (width 0.25) (layer "F.Cu") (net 3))
 (segment (start 178.64 93.64) (end 167.859 93.64) (width 0.25) (layer "F.Cu") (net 3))
 (segment (start 182.54 93.64) (end 182.88 93.98) (width 0.25) (layer "F.Cu") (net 3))
 (segment (start 178.64 93.64) (end 182.54 93.64) (width 0.25) (layer "F.Cu") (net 3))
 (segment (start 172.72 91.44) (end 168.199 91.44) (width 0.25) (layer "F.Cu") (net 2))
 (segment (start 168.199 91.44) (end 167.132 90.373) (width 0.25) (layer "F.Cu") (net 2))
 (segment (start 178.44 91.44) (end 178.64 91.64) (width 0.25) (layer "F.Cu") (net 2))
 (segment (start 172.72 91.44) (end 178.44 91.44) (width 0.25) (layer "F.Cu") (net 2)))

